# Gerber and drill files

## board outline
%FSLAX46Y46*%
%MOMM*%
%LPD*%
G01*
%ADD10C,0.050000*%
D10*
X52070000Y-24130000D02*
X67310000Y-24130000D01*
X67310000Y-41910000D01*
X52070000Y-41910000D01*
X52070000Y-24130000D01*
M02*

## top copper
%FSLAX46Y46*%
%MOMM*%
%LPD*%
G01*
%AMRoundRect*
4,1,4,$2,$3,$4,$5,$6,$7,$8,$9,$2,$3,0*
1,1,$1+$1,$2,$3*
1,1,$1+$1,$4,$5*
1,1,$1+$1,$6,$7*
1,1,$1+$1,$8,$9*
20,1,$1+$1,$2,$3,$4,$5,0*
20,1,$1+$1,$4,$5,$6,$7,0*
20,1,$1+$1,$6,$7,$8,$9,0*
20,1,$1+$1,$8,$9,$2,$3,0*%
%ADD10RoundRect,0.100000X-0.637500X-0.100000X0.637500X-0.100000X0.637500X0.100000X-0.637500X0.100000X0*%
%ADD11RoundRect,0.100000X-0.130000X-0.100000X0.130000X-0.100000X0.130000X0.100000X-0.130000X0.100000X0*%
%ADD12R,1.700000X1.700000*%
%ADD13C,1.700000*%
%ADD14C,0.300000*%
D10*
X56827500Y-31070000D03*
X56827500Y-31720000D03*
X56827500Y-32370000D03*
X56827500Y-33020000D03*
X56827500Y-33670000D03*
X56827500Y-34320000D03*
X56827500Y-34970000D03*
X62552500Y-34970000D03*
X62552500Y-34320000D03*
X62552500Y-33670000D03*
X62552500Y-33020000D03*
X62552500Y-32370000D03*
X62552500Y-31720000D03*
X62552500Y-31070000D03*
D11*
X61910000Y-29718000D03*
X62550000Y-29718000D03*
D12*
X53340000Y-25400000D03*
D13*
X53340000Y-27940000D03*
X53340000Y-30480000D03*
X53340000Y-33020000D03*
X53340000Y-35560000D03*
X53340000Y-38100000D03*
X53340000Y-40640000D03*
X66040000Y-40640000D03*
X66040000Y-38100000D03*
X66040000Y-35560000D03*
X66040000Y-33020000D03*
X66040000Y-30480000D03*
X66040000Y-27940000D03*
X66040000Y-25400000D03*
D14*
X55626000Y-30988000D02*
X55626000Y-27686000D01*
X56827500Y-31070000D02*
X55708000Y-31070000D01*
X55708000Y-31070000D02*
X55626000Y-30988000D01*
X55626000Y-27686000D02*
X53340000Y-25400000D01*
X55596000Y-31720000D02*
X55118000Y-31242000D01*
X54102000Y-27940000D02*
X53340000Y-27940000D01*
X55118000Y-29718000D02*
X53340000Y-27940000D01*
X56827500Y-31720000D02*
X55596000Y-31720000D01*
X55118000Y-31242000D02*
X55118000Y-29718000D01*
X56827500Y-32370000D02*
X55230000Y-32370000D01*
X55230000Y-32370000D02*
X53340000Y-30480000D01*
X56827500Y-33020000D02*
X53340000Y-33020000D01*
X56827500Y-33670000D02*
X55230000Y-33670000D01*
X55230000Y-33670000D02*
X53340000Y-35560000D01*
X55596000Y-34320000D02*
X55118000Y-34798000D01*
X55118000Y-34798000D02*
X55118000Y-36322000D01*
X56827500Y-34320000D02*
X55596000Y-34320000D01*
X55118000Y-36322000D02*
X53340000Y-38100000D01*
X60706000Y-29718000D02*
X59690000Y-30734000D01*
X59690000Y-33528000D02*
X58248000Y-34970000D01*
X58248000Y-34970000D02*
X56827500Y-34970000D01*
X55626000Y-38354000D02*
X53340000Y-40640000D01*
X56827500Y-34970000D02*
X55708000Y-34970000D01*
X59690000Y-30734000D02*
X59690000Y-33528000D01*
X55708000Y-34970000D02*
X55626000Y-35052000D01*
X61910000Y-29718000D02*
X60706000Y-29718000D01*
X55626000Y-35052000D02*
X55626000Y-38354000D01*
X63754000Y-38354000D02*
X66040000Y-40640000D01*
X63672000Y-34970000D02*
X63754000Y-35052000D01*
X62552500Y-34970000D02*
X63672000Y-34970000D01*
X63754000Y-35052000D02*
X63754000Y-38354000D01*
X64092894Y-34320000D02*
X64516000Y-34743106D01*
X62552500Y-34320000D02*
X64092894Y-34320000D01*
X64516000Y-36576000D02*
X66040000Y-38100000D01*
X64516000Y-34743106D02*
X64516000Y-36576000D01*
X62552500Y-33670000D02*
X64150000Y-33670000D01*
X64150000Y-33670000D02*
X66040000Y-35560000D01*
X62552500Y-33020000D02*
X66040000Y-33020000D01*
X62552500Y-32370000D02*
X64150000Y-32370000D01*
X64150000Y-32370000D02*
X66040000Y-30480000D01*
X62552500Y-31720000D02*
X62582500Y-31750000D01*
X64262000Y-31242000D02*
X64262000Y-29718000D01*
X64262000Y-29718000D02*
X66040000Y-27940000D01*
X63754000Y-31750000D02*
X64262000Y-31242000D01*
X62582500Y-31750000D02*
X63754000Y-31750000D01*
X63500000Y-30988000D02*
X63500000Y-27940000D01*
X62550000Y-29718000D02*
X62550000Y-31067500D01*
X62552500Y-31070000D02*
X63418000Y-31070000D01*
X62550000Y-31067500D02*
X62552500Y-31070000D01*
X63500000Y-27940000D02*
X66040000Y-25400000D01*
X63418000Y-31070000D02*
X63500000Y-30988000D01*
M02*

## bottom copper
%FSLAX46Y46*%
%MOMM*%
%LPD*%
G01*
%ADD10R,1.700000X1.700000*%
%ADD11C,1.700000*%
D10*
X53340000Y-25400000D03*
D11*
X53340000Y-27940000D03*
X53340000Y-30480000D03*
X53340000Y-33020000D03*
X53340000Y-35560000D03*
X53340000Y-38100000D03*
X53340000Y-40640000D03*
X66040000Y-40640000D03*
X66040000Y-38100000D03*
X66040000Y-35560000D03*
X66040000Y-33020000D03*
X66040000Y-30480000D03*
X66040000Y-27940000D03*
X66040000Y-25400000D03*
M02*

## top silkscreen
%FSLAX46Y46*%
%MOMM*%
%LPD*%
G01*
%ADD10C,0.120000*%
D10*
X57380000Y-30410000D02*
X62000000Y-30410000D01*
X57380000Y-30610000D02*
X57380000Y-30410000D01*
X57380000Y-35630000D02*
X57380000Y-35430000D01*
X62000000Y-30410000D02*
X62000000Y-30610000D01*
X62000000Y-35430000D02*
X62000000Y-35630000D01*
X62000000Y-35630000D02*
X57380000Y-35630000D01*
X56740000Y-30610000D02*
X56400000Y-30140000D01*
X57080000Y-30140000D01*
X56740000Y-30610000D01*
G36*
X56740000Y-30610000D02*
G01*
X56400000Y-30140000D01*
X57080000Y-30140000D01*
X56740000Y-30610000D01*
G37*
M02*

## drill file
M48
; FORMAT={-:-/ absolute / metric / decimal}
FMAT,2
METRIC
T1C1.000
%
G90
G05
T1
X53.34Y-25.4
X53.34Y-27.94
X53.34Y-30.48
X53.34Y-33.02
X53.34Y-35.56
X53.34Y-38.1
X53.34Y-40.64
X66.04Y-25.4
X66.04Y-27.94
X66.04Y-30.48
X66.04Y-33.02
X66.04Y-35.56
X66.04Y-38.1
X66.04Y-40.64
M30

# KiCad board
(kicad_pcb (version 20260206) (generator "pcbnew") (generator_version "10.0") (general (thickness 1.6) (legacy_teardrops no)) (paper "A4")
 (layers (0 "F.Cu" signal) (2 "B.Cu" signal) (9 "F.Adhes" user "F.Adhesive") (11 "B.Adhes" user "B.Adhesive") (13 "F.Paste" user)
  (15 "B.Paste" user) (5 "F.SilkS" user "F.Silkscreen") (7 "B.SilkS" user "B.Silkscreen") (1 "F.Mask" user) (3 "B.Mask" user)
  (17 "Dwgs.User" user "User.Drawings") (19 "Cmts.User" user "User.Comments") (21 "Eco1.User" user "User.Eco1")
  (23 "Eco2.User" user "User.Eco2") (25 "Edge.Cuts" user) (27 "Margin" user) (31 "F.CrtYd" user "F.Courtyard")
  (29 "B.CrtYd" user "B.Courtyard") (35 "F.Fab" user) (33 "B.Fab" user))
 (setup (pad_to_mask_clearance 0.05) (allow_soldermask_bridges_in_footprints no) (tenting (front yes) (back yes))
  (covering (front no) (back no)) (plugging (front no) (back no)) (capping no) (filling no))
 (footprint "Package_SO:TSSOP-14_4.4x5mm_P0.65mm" (layer "F.Cu") (at 59.69 33.02)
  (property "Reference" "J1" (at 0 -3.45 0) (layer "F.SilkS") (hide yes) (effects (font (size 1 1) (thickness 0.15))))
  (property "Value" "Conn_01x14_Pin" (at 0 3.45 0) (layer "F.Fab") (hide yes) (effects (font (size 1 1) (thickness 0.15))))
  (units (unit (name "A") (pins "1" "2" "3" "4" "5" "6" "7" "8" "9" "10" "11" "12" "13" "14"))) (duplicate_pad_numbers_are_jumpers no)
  (fp_line (start -2.31 -2.61) (end 2.31 -2.61) (stroke (width 0.12) (type solid)) (layer "F.SilkS"))
  (fp_line (start -2.31 -2.41) (end -2.31 -2.61) (stroke (width 0.12) (type solid)) (layer "F.SilkS"))
  (fp_line (start -2.31 2.61) (end -2.31 2.41) (stroke (width 0.12) (type solid)) (layer "F.SilkS"))
  (fp_line (start 2.31 -2.61) (end 2.31 -2.41) (stroke (width 0.12) (type solid)) (layer "F.SilkS"))
  (fp_line (start 2.31 2.41) (end 2.31 2.61) (stroke (width 0.12) (type solid)) (layer "F.SilkS"))
  (fp_line (start 2.31 2.61) (end -2.31 2.61) (stroke (width 0.12) (type solid)) (layer "F.SilkS"))
  (fp_poly (pts (xy -2.95 -2.41) (xy -3.29 -2.88) (xy -2.61 -2.88)) (stroke (width 0.12) (type solid)) (fill yes) (layer "F.SilkS"))
  (pad "1" smd roundrect (at -2.8625 -1.95) (size 1.475 0.4) (layers "F.Cu" "F.Mask" "F.Paste") (roundrect_rratio 0.25)
   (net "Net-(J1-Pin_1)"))
  (pad "2" smd roundrect (at -2.8625 -1.3) (size 1.475 0.4) (layers "F.Cu" "F.Mask" "F.Paste") (roundrect_rratio 0.25)
   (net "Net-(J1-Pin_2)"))
  (pad "3" smd roundrect (at -2.8625 -0.65) (size 1.475 0.4) (layers "F.Cu" "F.Mask" "F.Paste") (roundrect_rratio 0.25)
   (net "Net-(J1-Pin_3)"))
  (pad "4" smd roundrect (at -2.8625 0) (size 1.475 0.4) (layers "F.Cu" "F.Mask" "F.Paste") (roundrect_rratio 0.25) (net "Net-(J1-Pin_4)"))
  (pad "5" smd roundrect (at -2.8625 0.65) (size 1.475 0.4) (layers "F.Cu" "F.Mask" "F.Paste") (roundrect_rratio 0.25)
   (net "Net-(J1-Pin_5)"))
  (pad "6" smd roundrect (at -2.8625 1.3) (size 1.475 0.4) (layers "F.Cu" "F.Mask" "F.Paste") (roundrect_rratio 0.25) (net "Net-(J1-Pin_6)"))
  (pad "7" smd roundrect (at -2.8625 1.95) (size 1.475 0.4) (layers "F.Cu" "F.Mask" "F.Paste") (roundrect_rratio 0.25)
   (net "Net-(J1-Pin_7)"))
  (pad "8" smd roundrect (at 2.8625 1.95) (size 1.475 0.4) (layers "F.Cu" "F.Mask" "F.Paste") (roundrect_rratio 0.25) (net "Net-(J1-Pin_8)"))
  (pad "9" smd roundrect (at 2.8625 1.3) (size 1.475 0.4) (layers "F.Cu" "F.Mask" "F.Paste") (roundrect_rratio 0.25) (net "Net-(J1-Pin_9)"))
  (pad "10" smd roundrect (at 2.8625 0.65) (size 1.475 0.4) (layers "F.Cu" "F.Mask" "F.Paste") (roundrect_rratio 0.25)
   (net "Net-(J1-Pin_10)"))
  (pad "11" smd roundrect (at 2.8625 0) (size 1.475 0.4) (layers "F.Cu" "F.Mask" "F.Paste") (roundrect_rratio 0.25) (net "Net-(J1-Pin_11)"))
  (pad "12" smd roundrect (at 2.8625 -0.65) (size 1.475 0.4) (layers "F.Cu" "F.Mask" "F.Paste") (roundrect_rratio 0.25)
   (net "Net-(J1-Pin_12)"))
  (pad "13" smd roundrect (at 2.8625 -1.3) (size 1.475 0.4) (layers "F.Cu" "F.Mask" "F.Paste") (roundrect_rratio 0.25)
   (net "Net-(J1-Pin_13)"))
  (pad "14" smd roundrect (at 2.8625 -1.95) (size 1.475 0.4) (layers "F.Cu" "F.Mask" "F.Paste") (roundrect_rratio 0.25)
   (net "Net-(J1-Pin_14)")))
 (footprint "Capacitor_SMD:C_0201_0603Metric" (layer "F.Cu") (at 62.23 29.718)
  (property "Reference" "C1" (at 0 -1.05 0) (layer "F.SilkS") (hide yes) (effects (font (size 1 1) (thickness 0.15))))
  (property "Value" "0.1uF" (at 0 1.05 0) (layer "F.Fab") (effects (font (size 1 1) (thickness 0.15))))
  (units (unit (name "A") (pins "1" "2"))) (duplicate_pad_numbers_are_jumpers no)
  (pad "" smd roundrect (at -0.345 0) (size 0.318 0.36) (layers "F.Paste") (roundrect_rratio 0.25))
  (pad "" smd roundrect (at 0.345 0) (size 0.318 0.36) (layers "F.Paste") (roundrect_rratio 0.25))
  (pad "1" smd roundrect (at -0.32 0) (size 0.46 0.4) (layers "F.Cu" "F.Mask") (roundrect_rratio 0.25) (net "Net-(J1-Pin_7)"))
  (pad "2" smd roundrect (at 0.32 0) (size 0.46 0.4) (layers "F.Cu" "F.Mask") (roundrect_rratio 0.25) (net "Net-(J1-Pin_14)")))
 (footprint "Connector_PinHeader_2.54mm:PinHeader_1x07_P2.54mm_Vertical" (layer "B.Cu") (at 53.34 25.4 180)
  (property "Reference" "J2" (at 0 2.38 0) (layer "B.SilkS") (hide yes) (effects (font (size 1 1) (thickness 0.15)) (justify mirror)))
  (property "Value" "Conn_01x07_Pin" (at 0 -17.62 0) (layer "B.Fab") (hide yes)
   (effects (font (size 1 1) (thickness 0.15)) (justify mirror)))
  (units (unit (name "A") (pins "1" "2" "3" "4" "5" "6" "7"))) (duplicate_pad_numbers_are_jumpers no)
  (pad "1" thru_hole rect (at 0 0 180) (size 1.7 1.7) (drill 1) (layers "*.Cu" "*.Mask") (remove_unused_layers no) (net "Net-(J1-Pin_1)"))
  (pad "2" thru_hole circle (at 0 -2.54 180) (size 1.7 1.7) (drill 1) (layers "*.Cu" "*.Mask") (remove_unused_layers no)
   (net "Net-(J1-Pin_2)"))
  (pad "3" thru_hole circle (at 0 -5.08 180) (size 1.7 1.7) (drill 1) (layers "*.Cu" "*.Mask") (remove_unused_layers no)
   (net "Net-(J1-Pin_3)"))
  (pad "4" thru_hole circle (at 0 -7.62 180) (size 1.7 1.7) (drill 1) (layers "*.Cu" "*.Mask") (remove_unused_layers no)
   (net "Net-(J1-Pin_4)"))
  (pad "5" thru_hole circle (at 0 -10.16 180) (size 1.7 1.7) (drill 1) (layers "*.Cu" "*.Mask") (remove_unused_layers no)
   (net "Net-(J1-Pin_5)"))
  (pad "6" thru_hole circle (at 0 -12.7 180) (size 1.7 1.7) (drill 1) (layers "*.Cu" "*.Mask") (remove_unused_layers no)
   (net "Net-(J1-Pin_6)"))
  (pad "7" thru_hole circle (at 0 -15.24 180) (size 1.7 1.7) (drill 1) (layers "*.Cu" "*.Mask") (remove_unused_layers no)
   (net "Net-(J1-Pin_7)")))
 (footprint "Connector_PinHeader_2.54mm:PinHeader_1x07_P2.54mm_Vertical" (layer "B.Cu") (at 66.04 40.64)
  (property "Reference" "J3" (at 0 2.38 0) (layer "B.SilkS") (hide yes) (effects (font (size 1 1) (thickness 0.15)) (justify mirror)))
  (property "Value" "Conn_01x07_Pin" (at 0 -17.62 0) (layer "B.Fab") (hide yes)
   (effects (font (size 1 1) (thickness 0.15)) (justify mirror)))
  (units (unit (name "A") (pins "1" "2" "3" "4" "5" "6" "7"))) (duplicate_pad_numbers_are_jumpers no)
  (pad "1" thru_hole circle (at 0 0) (size 1.7 1.7) (drill 1) (layers "*.Cu" "*.Mask") (remove_unused_layers no) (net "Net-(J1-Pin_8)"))
  (pad "2" thru_hole circle (at 0 -2.54) (size 1.7 1.7) (drill 1) (layers "*.Cu" "*.Mask") (remove_unused_layers no) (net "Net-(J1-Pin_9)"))
  (pad "3" thru_hole circle (at 0 -5.08) (size 1.7 1.7) (drill 1) (layers "*.Cu" "*.Mask") (remove_unused_layers no) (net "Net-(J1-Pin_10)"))
  (pad "4" thru_hole circle (at 0 -7.62) (size 1.7 1.7) (drill 1) (layers "*.Cu" "*.Mask") (remove_unused_layers no) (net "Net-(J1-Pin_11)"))
  (pad "5" thru_hole circle (at 0 -10.16) (size 1.7 1.7) (drill 1) (layers "*.Cu" "*.Mask") (remove_unused_layers no)
   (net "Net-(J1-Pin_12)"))
  (pad "6" thru_hole circle (at 0 -12.7) (size 1.7 1.7) (drill 1) (layers "*.Cu" "*.Mask") (remove_unused_layers no) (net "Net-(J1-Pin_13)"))
  (pad "7" thru_hole circle (at 0 -15.24) (size 1.7 1.7) (drill 1) (layers "*.Cu" "*.Mask") (remove_unused_layers no)
   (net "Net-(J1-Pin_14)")))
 (gr_rect (start 52.07 24.13) (end 67.31 41.91) (stroke (width 0.05) (type default)) (fill no) (layer "Edge.Cuts"))
 (segment (start 55.626 30.988) (end 55.626 27.686) (width 0.3) (layer "F.Cu") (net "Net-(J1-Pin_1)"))
 (segment (start 56.8275 31.07) (end 55.708 31.07) (width 0.3) (layer "F.Cu") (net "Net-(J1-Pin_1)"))
 (segment (start 55.708 31.07) (end 55.626 30.988) (width 0.3) (layer "F.Cu") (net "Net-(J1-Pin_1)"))
 (segment (start 55.626 27.686) (end 53.34 25.4) (width 0.3) (layer "F.Cu") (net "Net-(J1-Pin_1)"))
 (segment (start 55.596 31.72) (end 55.118 31.242) (width 0.3) (layer "F.Cu") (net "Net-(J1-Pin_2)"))
 (segment (start 54.102 27.94) (end 53.34 27.94) (width 0.3) (layer "F.Cu") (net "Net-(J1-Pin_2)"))
 (segment (start 55.118 29.718) (end 53.34 27.94) (width 0.3) (layer "F.Cu") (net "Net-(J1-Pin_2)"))
 (segment (start 56.8275 31.72) (end 55.596 31.72) (width 0.3) (layer "F.Cu") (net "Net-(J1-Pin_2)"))
 (segment (start 55.118 31.242) (end 55.118 29.718) (width 0.3) (layer "F.Cu") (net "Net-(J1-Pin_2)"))
 (segment (start 56.8275 32.37) (end 55.23 32.37) (width 0.3) (layer "F.Cu") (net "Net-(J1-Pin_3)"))
 (segment (start 55.23 32.37) (end 53.34 30.48) (width 0.3) (layer "F.Cu") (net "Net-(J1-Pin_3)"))
 (segment (start 56.8275 33.02) (end 53.34 33.02) (width 0.3) (layer "F.Cu") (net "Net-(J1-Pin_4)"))
 (segment (start 56.8275 33.67) (end 55.23 33.67) (width 0.3) (layer "F.Cu") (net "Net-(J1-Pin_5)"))
 (segment (start 55.23 33.67) (end 53.34 35.56) (width 0.3) (layer "F.Cu") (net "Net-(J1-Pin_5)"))
 (segment (start 55.596 34.32) (end 55.118 34.798) (width 0.3) (layer "F.Cu") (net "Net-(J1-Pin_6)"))
 (segment (start 55.118 34.798) (end 55.118 36.322) (width 0.3) (layer "F.Cu") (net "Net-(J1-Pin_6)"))
 (segment (start 56.8275 34.32) (end 55.596 34.32) (width 0.3) (layer "F.Cu") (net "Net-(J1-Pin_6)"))
 (segment (start 55.118 36.322) (end 53.34 38.1) (width 0.3) (layer "F.Cu") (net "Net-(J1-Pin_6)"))
 (segment (start 60.706 29.718) (end 59.69 30.734) (width 0.3) (layer "F.Cu") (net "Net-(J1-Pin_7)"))
 (segment (start 59.69 33.528) (end 58.248 34.97) (width 0.3) (layer "F.Cu") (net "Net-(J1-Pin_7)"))
 (segment (start 58.248 34.97) (end 56.8275 34.97) (width 0.3) (layer "F.Cu") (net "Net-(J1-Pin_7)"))
 (segment (start 55.626 38.354) (end 53.34 40.64) (width 0.3) (layer "F.Cu") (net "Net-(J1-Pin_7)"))
 (segment (start 56.8275 34.97) (end 55.708 34.97) (width 0.3) (layer "F.Cu") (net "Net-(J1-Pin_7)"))
 (segment (start 59.69 30.734) (end 59.69 33.528) (width 0.3) (layer "F.Cu") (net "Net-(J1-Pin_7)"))
 (segment (start 55.708 34.97) (end 55.626 35.052) (width 0.3) (layer "F.Cu") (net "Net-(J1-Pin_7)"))
 (segment (start 61.91 29.718) (end 60.706 29.718) (width 0.3) (layer "F.Cu") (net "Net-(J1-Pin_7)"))
 (segment (start 55.626 35.052) (end 55.626 38.354) (width 0.3) (layer "F.Cu") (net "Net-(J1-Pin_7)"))
 (segment (start 63.754 38.354) (end 66.04 40.64) (width 0.3) (layer "F.Cu") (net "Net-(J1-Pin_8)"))
 (segment (start 63.672 34.97) (end 63.754 35.052) (width 0.3) (layer "F.Cu") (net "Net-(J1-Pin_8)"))
 (segment (start 62.5525 34.97) (end 63.672 34.97) (width 0.3) (layer "F.Cu") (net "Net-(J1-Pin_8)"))
 (segment (start 63.754 35.052) (end 63.754 38.354) (width 0.3) (layer "F.Cu") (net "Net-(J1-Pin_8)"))
 (segment (start 64.092894 34.32) (end 64.516 34.743106) (width 0.3) (layer "F.Cu") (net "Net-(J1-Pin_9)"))
 (segment (start 62.5525 34.32) (end 64.092894 34.32) (width 0.3) (layer "F.Cu") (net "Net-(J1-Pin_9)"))
 (segment (start 64.516 36.576) (end 66.04 38.1) (width 0.3) (layer "F.Cu") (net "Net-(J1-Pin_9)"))
 (segment (start 64.516 34.743106) (end 64.516 36.576) (width 0.3) (layer "F.Cu") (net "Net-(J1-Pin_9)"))
 (segment (start 62.5525 33.67) (end 64.15 33.67) (width 0.3) (layer "F.Cu") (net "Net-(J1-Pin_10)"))
 (segment (start 64.15 33.67) (end 66.04 35.56) (width 0.3) (layer "F.Cu") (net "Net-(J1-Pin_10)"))
 (segment (start 62.5525 33.02) (end 66.04 33.02) (width 0.3) (layer "F.Cu") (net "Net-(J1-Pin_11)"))
 (segment (start 62.5525 32.37) (end 64.15 32.37) (width 0.3) (layer "F.Cu") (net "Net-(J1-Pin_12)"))
 (segment (start 64.15 32.37) (end 66.04 30.48) (width 0.3) (layer "F.Cu") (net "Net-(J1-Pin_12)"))
 (segment (start 62.5525 31.72) (end 62.5825 31.75) (width 0.3) (layer "F.Cu") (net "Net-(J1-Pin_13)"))
 (segment (start 64.262 31.242) (end 64.262 29.718) (width 0.3) (layer "F.Cu") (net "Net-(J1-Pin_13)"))
 (segment (start 64.262 29.718) (end 66.04 27.94) (width 0.3) (layer "F.Cu") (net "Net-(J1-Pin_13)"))
 (segment (start 63.754 31.75) (end 64.262 31.242) (width 0.3) (layer "F.Cu") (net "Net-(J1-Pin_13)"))
 (segment (start 62.5825 31.75) (end 63.754 31.75) (width 0.3) (layer "F.Cu") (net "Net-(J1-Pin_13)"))
 (segment (start 63.5 30.988) (end 63.5 27.94) (width 0.3) (layer "F.Cu") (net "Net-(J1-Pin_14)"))
 (segment (start 62.55 29.718) (end 62.55 31.0675) (width 0.3) (layer "F.Cu") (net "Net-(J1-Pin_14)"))
 (segment (start 62.5525 31.07) (end 63.418 31.07) (width 0.3) (layer "F.Cu") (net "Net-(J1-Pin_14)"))
 (segment (start 62.55 31.0675) (end 62.5525 31.07) (width 0.3) (layer "F.Cu") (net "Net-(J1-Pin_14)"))
 (segment (start 63.5 27.94) (end 66.04 25.4) (width 0.3) (layer "F.Cu") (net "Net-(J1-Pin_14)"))
 (segment (start 63.418 31.07) (end 63.5 30.988) (width 0.3) (layer "F.Cu") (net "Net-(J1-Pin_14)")))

